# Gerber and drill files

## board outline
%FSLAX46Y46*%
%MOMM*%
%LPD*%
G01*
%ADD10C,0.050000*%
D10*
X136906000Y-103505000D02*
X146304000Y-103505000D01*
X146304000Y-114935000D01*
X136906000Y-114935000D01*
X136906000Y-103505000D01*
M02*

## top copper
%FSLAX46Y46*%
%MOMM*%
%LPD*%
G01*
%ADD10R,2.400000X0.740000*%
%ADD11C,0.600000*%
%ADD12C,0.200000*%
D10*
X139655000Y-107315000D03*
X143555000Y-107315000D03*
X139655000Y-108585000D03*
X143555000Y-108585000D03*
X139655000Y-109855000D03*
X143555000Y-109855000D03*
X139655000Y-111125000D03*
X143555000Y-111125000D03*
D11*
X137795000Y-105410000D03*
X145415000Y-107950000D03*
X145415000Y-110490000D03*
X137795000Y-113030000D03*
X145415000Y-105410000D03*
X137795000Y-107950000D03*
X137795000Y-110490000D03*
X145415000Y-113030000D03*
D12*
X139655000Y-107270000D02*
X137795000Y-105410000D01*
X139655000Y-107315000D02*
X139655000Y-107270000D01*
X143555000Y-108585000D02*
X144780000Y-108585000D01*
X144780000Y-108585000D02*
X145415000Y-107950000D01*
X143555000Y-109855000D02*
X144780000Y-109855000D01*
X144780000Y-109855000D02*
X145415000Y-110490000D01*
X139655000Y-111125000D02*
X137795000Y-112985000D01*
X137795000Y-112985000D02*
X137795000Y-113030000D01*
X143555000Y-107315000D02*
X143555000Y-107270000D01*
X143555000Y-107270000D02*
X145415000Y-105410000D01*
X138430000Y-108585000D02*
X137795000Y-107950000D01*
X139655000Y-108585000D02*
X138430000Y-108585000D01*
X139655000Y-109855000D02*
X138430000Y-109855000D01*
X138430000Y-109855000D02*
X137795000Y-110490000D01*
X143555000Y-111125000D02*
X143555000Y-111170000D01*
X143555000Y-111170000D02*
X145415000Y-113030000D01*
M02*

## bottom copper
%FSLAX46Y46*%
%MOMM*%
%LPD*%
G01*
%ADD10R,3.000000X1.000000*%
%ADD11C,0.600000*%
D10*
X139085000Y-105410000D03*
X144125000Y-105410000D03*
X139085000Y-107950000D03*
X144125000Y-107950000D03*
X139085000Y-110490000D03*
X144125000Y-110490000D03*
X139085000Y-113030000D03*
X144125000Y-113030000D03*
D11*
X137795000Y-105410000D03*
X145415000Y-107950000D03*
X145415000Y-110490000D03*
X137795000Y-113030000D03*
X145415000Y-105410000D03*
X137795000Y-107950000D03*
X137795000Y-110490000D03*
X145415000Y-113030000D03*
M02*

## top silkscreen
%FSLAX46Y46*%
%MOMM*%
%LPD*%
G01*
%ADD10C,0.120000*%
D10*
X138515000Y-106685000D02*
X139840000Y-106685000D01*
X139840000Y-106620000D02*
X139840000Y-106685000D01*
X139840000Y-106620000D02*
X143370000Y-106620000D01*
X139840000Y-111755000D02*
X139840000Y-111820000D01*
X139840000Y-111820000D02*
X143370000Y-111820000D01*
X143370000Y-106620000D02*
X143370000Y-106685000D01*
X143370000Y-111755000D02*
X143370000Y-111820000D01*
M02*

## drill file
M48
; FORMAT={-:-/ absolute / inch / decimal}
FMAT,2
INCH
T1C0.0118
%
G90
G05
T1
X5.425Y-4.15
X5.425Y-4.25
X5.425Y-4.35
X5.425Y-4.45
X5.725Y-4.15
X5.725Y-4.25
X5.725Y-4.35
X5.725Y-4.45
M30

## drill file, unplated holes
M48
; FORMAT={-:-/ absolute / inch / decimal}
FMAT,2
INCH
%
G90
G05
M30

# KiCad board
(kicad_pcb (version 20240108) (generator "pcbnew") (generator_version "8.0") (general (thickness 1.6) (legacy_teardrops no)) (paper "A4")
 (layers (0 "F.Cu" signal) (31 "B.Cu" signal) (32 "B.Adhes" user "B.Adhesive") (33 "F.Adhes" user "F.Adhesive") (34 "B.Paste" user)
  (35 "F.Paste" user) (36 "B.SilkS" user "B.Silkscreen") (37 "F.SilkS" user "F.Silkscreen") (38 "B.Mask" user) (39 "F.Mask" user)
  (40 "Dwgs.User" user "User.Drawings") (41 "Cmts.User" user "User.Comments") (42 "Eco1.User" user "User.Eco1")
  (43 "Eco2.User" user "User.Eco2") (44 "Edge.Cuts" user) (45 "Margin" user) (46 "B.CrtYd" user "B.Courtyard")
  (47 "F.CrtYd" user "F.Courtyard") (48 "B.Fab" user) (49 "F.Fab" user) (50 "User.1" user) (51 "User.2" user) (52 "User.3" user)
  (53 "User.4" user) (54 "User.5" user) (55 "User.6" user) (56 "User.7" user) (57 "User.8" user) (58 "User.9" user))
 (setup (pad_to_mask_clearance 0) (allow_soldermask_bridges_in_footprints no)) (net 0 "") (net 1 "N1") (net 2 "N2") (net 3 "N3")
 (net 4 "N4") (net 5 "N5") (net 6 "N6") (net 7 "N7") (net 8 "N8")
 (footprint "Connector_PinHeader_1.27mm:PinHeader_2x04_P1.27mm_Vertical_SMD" (layer "F.Cu") (at 141.605 109.22)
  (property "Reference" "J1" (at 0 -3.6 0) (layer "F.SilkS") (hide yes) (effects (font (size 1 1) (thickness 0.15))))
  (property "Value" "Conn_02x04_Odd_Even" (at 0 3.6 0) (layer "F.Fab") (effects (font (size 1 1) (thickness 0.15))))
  (fp_line (start -3.09 -2.535) (end -1.765 -2.535) (stroke (width 0.12) (type solid)) (layer "F.SilkS"))
  (fp_line (start -1.765 -2.6) (end -1.765 -2.535) (stroke (width 0.12) (type solid)) (layer "F.SilkS"))
  (fp_line (start -1.765 -2.6) (end 1.765 -2.6) (stroke (width 0.12) (type solid)) (layer "F.SilkS"))
  (fp_line (start -1.765 2.535) (end -1.765 2.6) (stroke (width 0.12) (type solid)) (layer "F.SilkS"))
  (fp_line (start -1.765 2.6) (end 1.765 2.6) (stroke (width 0.12) (type solid)) (layer "F.SilkS"))
  (fp_line (start 1.765 -2.6) (end 1.765 -2.535) (stroke (width 0.12) (type solid)) (layer "F.SilkS"))
  (fp_line (start 1.765 2.535) (end 1.765 2.6) (stroke (width 0.12) (type solid)) (layer "F.SilkS"))
  (pad "1" smd rect (at -1.95 -1.905) (size 2.4 0.74) (layers "F.Cu" "F.Paste" "F.Mask") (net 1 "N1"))
  (pad "2" smd rect (at 1.95 -1.905) (size 2.4 0.74) (layers "F.Cu" "F.Paste" "F.Mask") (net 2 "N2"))
  (pad "3" smd rect (at -1.95 -0.635) (size 2.4 0.74) (layers "F.Cu" "F.Paste" "F.Mask") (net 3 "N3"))
  (pad "4" smd rect (at 1.95 -0.635) (size 2.4 0.74) (layers "F.Cu" "F.Paste" "F.Mask") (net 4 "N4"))
  (pad "5" smd rect (at -1.95 0.635) (size 2.4 0.74) (layers "F.Cu" "F.Paste" "F.Mask") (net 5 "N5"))
  (pad "6" smd rect (at 1.95 0.635) (size 2.4 0.74) (layers "F.Cu" "F.Paste" "F.Mask") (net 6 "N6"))
  (pad "7" smd rect (at -1.95 1.905) (size 2.4 0.74) (layers "F.Cu" "F.Paste" "F.Mask") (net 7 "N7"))
  (pad "8" smd rect (at 1.95 1.905) (size 2.4 0.74) (layers "F.Cu" "F.Paste" "F.Mask") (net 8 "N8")))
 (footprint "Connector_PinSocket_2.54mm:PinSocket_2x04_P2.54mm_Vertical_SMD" (layer "B.Cu") (at 141.605 109.22 180)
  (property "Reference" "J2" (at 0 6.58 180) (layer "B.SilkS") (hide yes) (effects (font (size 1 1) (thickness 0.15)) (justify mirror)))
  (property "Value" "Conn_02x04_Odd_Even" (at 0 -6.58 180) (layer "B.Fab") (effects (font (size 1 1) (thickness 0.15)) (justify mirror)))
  (pad "1" smd rect (at 2.52 3.81 180) (size 3 1) (layers "B.Cu" "B.Paste" "B.Mask") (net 1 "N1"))
  (pad "2" smd rect (at -2.52 3.81 180) (size 3 1) (layers "B.Cu" "B.Paste" "B.Mask") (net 2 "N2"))
  (pad "3" smd rect (at 2.52 1.27 180) (size 3 1) (layers "B.Cu" "B.Paste" "B.Mask") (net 3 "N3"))
  (pad "4" smd rect (at -2.52 1.27 180) (size 3 1) (layers "B.Cu" "B.Paste" "B.Mask") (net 4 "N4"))
  (pad "5" smd rect (at 2.52 -1.27 180) (size 3 1) (layers "B.Cu" "B.Paste" "B.Mask") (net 5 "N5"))
  (pad "6" smd rect (at -2.52 -1.27 180) (size 3 1) (layers "B.Cu" "B.Paste" "B.Mask") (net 6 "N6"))
  (pad "7" smd rect (at 2.52 -3.81 180) (size 3 1) (layers "B.Cu" "B.Paste" "B.Mask") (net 7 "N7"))
  (pad "8" smd rect (at -2.52 -3.81 180) (size 3 1) (layers "B.Cu" "B.Paste" "B.Mask") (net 8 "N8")))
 (gr_rect (start 136.906 103.505) (end 146.304 114.935) (stroke (width 0.05) (type default)) (fill none) (layer "Edge.Cuts"))
 (segment (start 139.655 107.27) (end 137.795 105.41) (width 0.2) (layer "F.Cu") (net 1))
 (segment (start 139.655 107.315) (end 139.655 107.27) (width 0.2) (layer "F.Cu") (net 1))
 (via (at 137.795 105.41) (size 0.6) (drill 0.3) (layers "F.Cu" "B.Cu") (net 1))
 (segment (start 143.555 108.585) (end 144.78 108.585) (width 0.2) (layer "F.Cu") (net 4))
 (segment (start 144.78 108.585) (end 145.415 107.95) (width 0.2) (layer "F.Cu") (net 4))
 (via (at 145.415 107.95) (size 0.6) (drill 0.3) (layers "F.Cu" "B.Cu") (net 4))
 (segment (start 143.555 109.855) (end 144.78 109.855) (width 0.2) (layer "F.Cu") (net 6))
 (segment (start 144.78 109.855) (end 145.415 110.49) (width 0.2) (layer "F.Cu") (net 6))
 (via (at 145.415 110.49) (size 0.6) (drill 0.3) (layers "F.Cu" "B.Cu") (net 6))
 (segment (start 139.655 111.125) (end 137.795 112.985) (width 0.2) (layer "F.Cu") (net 7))
 (segment (start 137.795 112.985) (end 137.795 113.03) (width 0.2) (layer "F.Cu") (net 7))
 (via (at 137.795 113.03) (size 0.6) (drill 0.3) (layers "F.Cu" "B.Cu") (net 7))
 (segment (start 143.555 107.315) (end 143.555 107.27) (width 0.2) (layer "F.Cu") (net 2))
 (segment (start 143.555 107.27) (end 145.415 105.41) (width 0.2) (layer "F.Cu") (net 2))
 (via (at 145.415 105.41) (size 0.6) (drill 0.3) (layers "F.Cu" "B.Cu") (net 2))
 (segment (start 138.43 108.585) (end 137.795 107.95) (width 0.2) (layer "F.Cu") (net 3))
 (segment (start 139.655 108.585) (end 138.43 108.585) (width 0.2) (layer "F.Cu") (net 3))
 (via (at 137.795 107.95) (size 0.6) (drill 0.3) (layers "F.Cu" "B.Cu") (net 3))
 (segment (start 139.655 109.855) (end 138.43 109.855) (width 0.2) (layer "F.Cu") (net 5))
 (segment (start 138.43 109.855) (end 137.795 110.49) (width 0.2) (layer "F.Cu") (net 5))
 (via (at 137.795 110.49) (size 0.6) (drill 0.3) (layers "F.Cu" "B.Cu") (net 5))
 (segment (start 143.555 111.125) (end 143.555 111.17) (width 0.2) (layer "F.Cu") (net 8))
 (segment (start 143.555 111.17) (end 145.415 113.03) (width 0.2) (layer "F.Cu") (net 8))
 (via (at 145.415 113.03) (size 0.6) (drill 0.3) (layers "F.Cu" "B.Cu") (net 8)))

